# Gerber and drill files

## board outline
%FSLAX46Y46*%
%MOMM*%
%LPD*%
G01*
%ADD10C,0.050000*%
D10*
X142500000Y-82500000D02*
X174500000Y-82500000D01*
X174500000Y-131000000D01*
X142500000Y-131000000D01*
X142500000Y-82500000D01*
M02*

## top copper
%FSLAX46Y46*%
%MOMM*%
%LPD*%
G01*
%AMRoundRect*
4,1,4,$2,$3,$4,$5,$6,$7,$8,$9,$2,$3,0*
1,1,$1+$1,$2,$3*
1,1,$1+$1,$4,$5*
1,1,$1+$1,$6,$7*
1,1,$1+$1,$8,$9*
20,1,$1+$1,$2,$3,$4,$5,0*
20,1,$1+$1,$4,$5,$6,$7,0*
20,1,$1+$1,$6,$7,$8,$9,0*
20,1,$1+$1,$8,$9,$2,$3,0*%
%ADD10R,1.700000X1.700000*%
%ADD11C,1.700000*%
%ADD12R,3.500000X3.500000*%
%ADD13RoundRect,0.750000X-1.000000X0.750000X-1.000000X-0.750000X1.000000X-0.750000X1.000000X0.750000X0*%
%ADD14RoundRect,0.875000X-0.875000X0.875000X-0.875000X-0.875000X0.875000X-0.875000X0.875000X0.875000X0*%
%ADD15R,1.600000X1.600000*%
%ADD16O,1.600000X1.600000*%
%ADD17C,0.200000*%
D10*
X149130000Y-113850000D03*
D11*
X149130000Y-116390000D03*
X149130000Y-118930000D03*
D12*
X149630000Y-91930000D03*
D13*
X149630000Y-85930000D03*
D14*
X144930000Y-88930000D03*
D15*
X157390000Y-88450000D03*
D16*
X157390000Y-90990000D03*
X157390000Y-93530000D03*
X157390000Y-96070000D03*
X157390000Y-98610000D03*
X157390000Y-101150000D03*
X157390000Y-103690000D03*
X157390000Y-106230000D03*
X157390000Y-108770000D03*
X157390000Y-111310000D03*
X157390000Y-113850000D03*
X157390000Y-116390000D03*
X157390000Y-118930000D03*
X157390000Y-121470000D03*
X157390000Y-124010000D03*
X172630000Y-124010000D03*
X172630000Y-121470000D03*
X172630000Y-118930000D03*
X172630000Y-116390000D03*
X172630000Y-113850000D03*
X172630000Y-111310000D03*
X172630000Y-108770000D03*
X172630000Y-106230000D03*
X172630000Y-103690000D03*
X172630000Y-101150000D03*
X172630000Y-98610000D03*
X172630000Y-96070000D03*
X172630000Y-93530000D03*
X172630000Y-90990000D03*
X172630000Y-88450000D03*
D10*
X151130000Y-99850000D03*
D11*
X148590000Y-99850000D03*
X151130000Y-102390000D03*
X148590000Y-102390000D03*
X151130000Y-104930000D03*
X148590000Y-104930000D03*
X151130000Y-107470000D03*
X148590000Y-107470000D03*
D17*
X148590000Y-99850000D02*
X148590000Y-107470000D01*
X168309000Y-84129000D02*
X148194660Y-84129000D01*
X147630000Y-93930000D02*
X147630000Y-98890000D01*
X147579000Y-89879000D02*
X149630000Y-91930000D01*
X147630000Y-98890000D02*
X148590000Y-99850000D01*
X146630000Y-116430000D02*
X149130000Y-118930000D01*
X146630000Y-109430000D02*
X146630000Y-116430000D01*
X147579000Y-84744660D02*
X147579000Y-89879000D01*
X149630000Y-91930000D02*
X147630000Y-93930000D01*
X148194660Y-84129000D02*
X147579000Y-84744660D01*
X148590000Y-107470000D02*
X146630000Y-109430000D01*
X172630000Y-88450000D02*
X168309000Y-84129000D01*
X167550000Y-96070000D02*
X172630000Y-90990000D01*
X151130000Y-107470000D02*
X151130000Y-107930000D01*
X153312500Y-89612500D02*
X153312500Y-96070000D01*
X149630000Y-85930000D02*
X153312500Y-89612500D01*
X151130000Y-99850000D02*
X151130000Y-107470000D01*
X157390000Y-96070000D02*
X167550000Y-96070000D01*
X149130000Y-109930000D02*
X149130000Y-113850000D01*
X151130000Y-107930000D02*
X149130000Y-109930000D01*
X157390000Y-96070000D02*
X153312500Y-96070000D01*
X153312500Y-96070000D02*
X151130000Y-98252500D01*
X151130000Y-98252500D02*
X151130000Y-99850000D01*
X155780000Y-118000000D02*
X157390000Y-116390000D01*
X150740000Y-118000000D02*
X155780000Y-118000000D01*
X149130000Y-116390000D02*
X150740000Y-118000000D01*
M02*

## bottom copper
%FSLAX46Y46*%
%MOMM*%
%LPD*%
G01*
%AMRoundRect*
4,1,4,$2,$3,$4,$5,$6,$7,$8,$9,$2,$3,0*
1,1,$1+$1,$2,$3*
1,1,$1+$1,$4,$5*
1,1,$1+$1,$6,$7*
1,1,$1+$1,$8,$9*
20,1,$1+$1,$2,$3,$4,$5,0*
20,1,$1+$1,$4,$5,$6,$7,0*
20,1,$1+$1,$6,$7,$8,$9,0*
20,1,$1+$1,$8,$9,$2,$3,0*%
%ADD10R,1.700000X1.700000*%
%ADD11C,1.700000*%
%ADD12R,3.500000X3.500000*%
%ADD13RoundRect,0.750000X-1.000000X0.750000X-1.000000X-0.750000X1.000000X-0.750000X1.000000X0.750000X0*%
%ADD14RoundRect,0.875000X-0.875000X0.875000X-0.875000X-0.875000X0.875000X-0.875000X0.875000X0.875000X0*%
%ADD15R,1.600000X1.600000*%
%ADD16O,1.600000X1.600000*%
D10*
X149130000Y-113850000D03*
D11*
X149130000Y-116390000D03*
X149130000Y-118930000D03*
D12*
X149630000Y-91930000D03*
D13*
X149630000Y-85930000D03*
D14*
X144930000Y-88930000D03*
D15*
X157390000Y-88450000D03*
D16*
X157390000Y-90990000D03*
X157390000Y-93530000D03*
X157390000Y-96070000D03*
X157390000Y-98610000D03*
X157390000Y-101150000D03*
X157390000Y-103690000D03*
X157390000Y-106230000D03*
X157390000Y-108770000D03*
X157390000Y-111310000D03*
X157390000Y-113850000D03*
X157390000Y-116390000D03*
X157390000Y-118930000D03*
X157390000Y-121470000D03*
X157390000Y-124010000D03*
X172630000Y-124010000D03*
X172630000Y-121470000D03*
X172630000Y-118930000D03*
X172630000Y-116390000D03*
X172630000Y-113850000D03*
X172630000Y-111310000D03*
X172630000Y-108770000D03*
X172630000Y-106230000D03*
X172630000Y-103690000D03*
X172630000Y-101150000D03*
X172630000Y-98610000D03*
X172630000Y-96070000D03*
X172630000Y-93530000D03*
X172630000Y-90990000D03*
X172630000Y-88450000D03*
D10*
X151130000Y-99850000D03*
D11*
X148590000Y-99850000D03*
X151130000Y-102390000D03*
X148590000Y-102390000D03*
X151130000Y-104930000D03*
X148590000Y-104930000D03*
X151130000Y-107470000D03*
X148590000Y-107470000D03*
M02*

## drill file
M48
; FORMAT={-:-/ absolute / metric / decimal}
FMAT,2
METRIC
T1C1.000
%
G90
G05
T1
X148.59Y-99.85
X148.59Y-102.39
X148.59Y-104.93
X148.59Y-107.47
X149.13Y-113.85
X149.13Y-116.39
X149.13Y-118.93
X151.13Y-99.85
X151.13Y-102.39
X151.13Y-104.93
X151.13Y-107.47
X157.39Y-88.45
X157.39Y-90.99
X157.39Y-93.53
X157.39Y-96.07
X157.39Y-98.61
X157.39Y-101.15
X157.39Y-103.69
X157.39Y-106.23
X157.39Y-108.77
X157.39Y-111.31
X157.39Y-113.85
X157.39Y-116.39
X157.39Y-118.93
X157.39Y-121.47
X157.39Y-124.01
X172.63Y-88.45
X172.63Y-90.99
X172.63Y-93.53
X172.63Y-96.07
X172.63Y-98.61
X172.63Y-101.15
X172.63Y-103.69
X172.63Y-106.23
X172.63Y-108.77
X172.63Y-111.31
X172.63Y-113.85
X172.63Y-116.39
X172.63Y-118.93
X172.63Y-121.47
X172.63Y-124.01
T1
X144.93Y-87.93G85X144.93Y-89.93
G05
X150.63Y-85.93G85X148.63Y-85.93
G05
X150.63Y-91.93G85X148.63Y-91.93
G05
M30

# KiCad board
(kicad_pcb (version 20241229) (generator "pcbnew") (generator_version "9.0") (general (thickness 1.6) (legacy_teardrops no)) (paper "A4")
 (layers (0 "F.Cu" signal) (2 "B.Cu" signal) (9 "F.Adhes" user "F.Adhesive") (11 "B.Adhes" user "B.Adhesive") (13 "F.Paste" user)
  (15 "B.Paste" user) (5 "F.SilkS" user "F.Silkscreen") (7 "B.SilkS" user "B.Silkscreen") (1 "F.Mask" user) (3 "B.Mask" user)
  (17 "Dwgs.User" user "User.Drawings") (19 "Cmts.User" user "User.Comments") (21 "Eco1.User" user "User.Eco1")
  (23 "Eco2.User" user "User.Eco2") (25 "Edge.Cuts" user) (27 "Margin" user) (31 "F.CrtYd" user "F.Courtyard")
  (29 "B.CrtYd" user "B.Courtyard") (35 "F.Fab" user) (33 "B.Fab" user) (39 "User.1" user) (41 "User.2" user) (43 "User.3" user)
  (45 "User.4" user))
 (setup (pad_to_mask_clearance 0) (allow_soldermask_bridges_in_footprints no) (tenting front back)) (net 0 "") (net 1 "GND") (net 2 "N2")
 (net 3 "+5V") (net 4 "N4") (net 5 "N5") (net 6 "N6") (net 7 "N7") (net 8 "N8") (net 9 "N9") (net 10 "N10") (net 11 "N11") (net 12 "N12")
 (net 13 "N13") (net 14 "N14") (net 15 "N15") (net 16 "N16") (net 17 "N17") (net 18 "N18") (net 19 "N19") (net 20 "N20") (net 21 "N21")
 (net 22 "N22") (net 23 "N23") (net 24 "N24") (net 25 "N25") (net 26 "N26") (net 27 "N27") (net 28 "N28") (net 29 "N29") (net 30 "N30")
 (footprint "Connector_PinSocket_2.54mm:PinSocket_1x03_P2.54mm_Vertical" (layer "F.Cu") (at 149.13 113.85)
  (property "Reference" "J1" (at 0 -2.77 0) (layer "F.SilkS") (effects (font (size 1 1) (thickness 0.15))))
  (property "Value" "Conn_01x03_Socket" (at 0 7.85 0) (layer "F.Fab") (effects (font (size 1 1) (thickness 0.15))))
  (pad "1" thru_hole rect (at 0 0) (size 1.7 1.7) (drill 1) (layers "*.Cu" "*.Mask") (remove_unused_layers no) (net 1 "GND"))
  (pad "2" thru_hole circle (at 0 2.54) (size 1.7 1.7) (drill 1) (layers "*.Cu" "*.Mask") (remove_unused_layers no) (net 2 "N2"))
  (pad "3" thru_hole circle (at 0 5.08) (size 1.7 1.7) (drill 1) (layers "*.Cu" "*.Mask") (remove_unused_layers no) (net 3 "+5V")))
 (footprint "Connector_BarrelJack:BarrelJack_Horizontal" (layer "F.Cu") (at 149.63 91.93 -90)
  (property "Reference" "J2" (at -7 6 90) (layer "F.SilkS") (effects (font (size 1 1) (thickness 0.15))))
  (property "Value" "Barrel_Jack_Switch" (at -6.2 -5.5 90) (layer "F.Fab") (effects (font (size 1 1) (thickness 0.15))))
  (pad "1" thru_hole rect (at 0 0 270) (size 3.5 3.5) (drill oval 1 3) (layers "*.Cu" "*.Mask") (remove_unused_layers no) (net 3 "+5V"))
  (pad "2" thru_hole roundrect (at -6 0 270) (size 3 3.5) (drill oval 1 3) (layers "*.Cu" "*.Mask") (remove_unused_layers no)
   (roundrect_rratio 0.25) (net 1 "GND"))
  (pad "3" thru_hole roundrect (at -3 4.7 270) (size 3.5 3.5) (drill oval 3 1) (layers "*.Cu" "*.Mask") (remove_unused_layers no)
   (roundrect_rratio 0.25) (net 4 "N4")))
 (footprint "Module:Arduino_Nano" (layer "F.Cu") (at 157.39 88.45)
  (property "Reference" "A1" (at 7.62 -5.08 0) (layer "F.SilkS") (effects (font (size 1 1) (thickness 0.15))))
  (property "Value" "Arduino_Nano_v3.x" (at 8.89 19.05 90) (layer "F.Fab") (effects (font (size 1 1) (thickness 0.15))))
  (pad "1" thru_hole rect (at 0 0) (size 1.6 1.6) (drill 1) (layers "*.Cu" "*.Mask") (remove_unused_layers no) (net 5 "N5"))
  (pad "2" thru_hole oval (at 0 2.54) (size 1.6 1.6) (drill 1) (layers "*.Cu" "*.Mask") (remove_unused_layers no) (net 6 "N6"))
  (pad "3" thru_hole oval (at 0 5.08) (size 1.6 1.6) (drill 1) (layers "*.Cu" "*.Mask") (remove_unused_layers no) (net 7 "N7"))
  (pad "4" thru_hole oval (at 0 7.62) (size 1.6 1.6) (drill 1) (layers "*.Cu" "*.Mask") (remove_unused_layers no) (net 1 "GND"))
  (pad "5" thru_hole oval (at 0 10.16) (size 1.6 1.6) (drill 1) (layers "*.Cu" "*.Mask") (remove_unused_layers no) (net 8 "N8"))
  (pad "6" thru_hole oval (at 0 12.7) (size 1.6 1.6) (drill 1) (layers "*.Cu" "*.Mask") (remove_unused_layers no) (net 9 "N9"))
  (pad "7" thru_hole oval (at 0 15.24) (size 1.6 1.6) (drill 1) (layers "*.Cu" "*.Mask") (remove_unused_layers no) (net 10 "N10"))
  (pad "8" thru_hole oval (at 0 17.78) (size 1.6 1.6) (drill 1) (layers "*.Cu" "*.Mask") (remove_unused_layers no) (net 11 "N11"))
  (pad "9" thru_hole oval (at 0 20.32) (size 1.6 1.6) (drill 1) (layers "*.Cu" "*.Mask") (remove_unused_layers no) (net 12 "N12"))
  (pad "10" thru_hole oval (at 0 22.86) (size 1.6 1.6) (drill 1) (layers "*.Cu" "*.Mask") (remove_unused_layers no) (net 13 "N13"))
  (pad "11" thru_hole oval (at 0 25.4) (size 1.6 1.6) (drill 1) (layers "*.Cu" "*.Mask") (remove_unused_layers no) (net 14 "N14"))
  (pad "12" thru_hole oval (at 0 27.94) (size 1.6 1.6) (drill 1) (layers "*.Cu" "*.Mask") (remove_unused_layers no) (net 2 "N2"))
  (pad "13" thru_hole oval (at 0 30.48) (size 1.6 1.6) (drill 1) (layers "*.Cu" "*.Mask") (remove_unused_layers no) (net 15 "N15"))
  (pad "14" thru_hole oval (at 0 33.02) (size 1.6 1.6) (drill 1) (layers "*.Cu" "*.Mask") (remove_unused_layers no) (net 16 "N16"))
  (pad "15" thru_hole oval (at 0 35.56) (size 1.6 1.6) (drill 1) (layers "*.Cu" "*.Mask") (remove_unused_layers no) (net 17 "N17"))
  (pad "16" thru_hole oval (at 15.24 35.56) (size 1.6 1.6) (drill 1) (layers "*.Cu" "*.Mask") (remove_unused_layers no) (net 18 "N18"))
  (pad "17" thru_hole oval (at 15.24 33.02) (size 1.6 1.6) (drill 1) (layers "*.Cu" "*.Mask") (remove_unused_layers no) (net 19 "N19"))
  (pad "18" thru_hole oval (at 15.24 30.48) (size 1.6 1.6) (drill 1) (layers "*.Cu" "*.Mask") (remove_unused_layers no) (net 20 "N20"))
  (pad "19" thru_hole oval (at 15.24 27.94) (size 1.6 1.6) (drill 1) (layers "*.Cu" "*.Mask") (remove_unused_layers no) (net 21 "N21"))
  (pad "20" thru_hole oval (at 15.24 25.4) (size 1.6 1.6) (drill 1) (layers "*.Cu" "*.Mask") (remove_unused_layers no) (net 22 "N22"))
  (pad "21" thru_hole oval (at 15.24 22.86) (size 1.6 1.6) (drill 1) (layers "*.Cu" "*.Mask") (remove_unused_layers no) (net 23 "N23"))
  (pad "22" thru_hole oval (at 15.24 20.32) (size 1.6 1.6) (drill 1) (layers "*.Cu" "*.Mask") (remove_unused_layers no) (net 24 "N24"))
  (pad "23" thru_hole oval (at 15.24 17.78) (size 1.6 1.6) (drill 1) (layers "*.Cu" "*.Mask") (remove_unused_layers no) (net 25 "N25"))
  (pad "24" thru_hole oval (at 15.24 15.24) (size 1.6 1.6) (drill 1) (layers "*.Cu" "*.Mask") (remove_unused_layers no) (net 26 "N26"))
  (pad "25" thru_hole oval (at 15.24 12.7) (size 1.6 1.6) (drill 1) (layers "*.Cu" "*.Mask") (remove_unused_layers no) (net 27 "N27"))
  (pad "26" thru_hole oval (at 15.24 10.16) (size 1.6 1.6) (drill 1) (layers "*.Cu" "*.Mask") (remove_unused_layers no) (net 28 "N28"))
  (pad "27" thru_hole oval (at 15.24 7.62) (size 1.6 1.6) (drill 1) (layers "*.Cu" "*.Mask") (remove_unused_layers no) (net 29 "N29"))
  (pad "28" thru_hole oval (at 15.24 5.08) (size 1.6 1.6) (drill 1) (layers "*.Cu" "*.Mask") (remove_unused_layers no) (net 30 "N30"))
  (pad "29" thru_hole oval (at 15.24 2.54) (size 1.6 1.6) (drill 1) (layers "*.Cu" "*.Mask") (remove_unused_layers no) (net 1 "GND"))
  (pad "30" thru_hole oval (at 15.24 0) (size 1.6 1.6) (drill 1) (layers "*.Cu" "*.Mask") (remove_unused_layers no) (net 3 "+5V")))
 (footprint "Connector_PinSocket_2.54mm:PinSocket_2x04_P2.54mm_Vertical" (layer "F.Cu") (at 151.13 99.85)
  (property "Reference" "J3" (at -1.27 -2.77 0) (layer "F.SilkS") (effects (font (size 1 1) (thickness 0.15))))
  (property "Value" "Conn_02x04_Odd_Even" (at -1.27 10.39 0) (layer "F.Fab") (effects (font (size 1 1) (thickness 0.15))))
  (pad "1" thru_hole rect (at 0 0) (size 1.7 1.7) (drill 1) (layers "*.Cu" "*.Mask") (remove_unused_layers no) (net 1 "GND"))
  (pad "2" thru_hole circle (at -2.54 0) (size 1.7 1.7) (drill 1) (layers "*.Cu" "*.Mask") (remove_unused_layers no) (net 3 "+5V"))
  (pad "3" thru_hole circle (at 0 2.54) (size 1.7 1.7) (drill 1) (layers "*.Cu" "*.Mask") (remove_unused_layers no) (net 1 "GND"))
  (pad "4" thru_hole circle (at -2.54 2.54) (size 1.7 1.7) (drill 1) (layers "*.Cu" "*.Mask") (remove_unused_layers no) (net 3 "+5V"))
  (pad "5" thru_hole circle (at 0 5.08) (size 1.7 1.7) (drill 1) (layers "*.Cu" "*.Mask") (remove_unused_layers no) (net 1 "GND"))
  (pad "6" thru_hole circle (at -2.54 5.08) (size 1.7 1.7) (drill 1) (layers "*.Cu" "*.Mask") (remove_unused_layers no) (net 3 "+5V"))
  (pad "7" thru_hole circle (at 0 7.62) (size 1.7 1.7) (drill 1) (layers "*.Cu" "*.Mask") (remove_unused_layers no) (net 1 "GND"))
  (pad "8" thru_hole circle (at -2.54 7.62) (size 1.7 1.7) (drill 1) (layers "*.Cu" "*.Mask") (remove_unused_layers no) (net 3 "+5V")))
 (gr_rect (start 142.5 82.5) (end 174.5 131) (stroke (width 0.05) (type default)) (fill no) (layer "Edge.Cuts"))
 (segment (start 148.59 99.85) (end 148.59 107.47) (width 0.2) (layer "F.Cu") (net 3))
 (segment (start 168.309 84.129) (end 148.19466 84.129) (width 0.2) (layer "F.Cu") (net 3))
 (segment (start 147.63 93.93) (end 147.63 98.89) (width 0.2) (layer "F.Cu") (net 3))
 (segment (start 147.579 89.879) (end 149.63 91.93) (width 0.2) (layer "F.Cu") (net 3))
 (segment (start 147.63 98.89) (end 148.59 99.85) (width 0.2) (layer "F.Cu") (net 3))
 (segment (start 146.63 116.43) (end 149.13 118.93) (width 0.2) (layer "F.Cu") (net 3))
 (segment (start 146.63 109.43) (end 146.63 116.43) (width 0.2) (layer "F.Cu") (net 3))
 (segment (start 147.579 84.74466) (end 147.579 89.879) (width 0.2) (layer "F.Cu") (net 3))
 (segment (start 149.63 91.93) (end 147.63 93.93) (width 0.2) (layer "F.Cu") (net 3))
 (segment (start 148.19466 84.129) (end 147.579 84.74466) (width 0.2) (layer "F.Cu") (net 3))
 (segment (start 148.59 107.47) (end 146.63 109.43) (width 0.2) (layer "F.Cu") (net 3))
 (segment (start 172.63 88.45) (end 168.309 84.129) (width 0.2) (layer "F.Cu") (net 3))
 (segment (start 167.55 96.07) (end 172.63 90.99) (width 0.2) (layer "F.Cu") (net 1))
 (segment (start 151.13 107.47) (end 151.13 107.93) (width 0.2) (layer "F.Cu") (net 1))
 (segment (start 153.3125 89.6125) (end 153.3125 96.07) (width 0.2) (layer "F.Cu") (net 1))
 (segment (start 149.63 85.93) (end 153.3125 89.6125) (width 0.2) (layer "F.Cu") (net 1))
 (segment (start 151.13 99.85) (end 151.13 107.47) (width 0.2) (layer "F.Cu") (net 1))
 (segment (start 157.39 96.07) (end 167.55 96.07) (width 0.2) (layer "F.Cu") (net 1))
 (segment (start 149.13 109.93) (end 149.13 113.85) (width 0.2) (layer "F.Cu") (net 1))
 (segment (start 151.13 107.93) (end 149.13 109.93) (width 0.2) (layer "F.Cu") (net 1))
 (segment (start 157.39 96.07) (end 153.3125 96.07) (width 0.2) (layer "F.Cu") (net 1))
 (segment (start 153.3125 96.07) (end 151.13 98.2525) (width 0.2) (layer "F.Cu") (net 1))
 (segment (start 151.13 98.2525) (end 151.13 99.85) (width 0.2) (layer "F.Cu") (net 1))
 (segment (start 155.78 118) (end 157.39 116.39) (width 0.2) (layer "F.Cu") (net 2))
 (segment (start 150.74 118) (end 155.78 118) (width 0.2) (layer "F.Cu") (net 2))
 (segment (start 149.13 116.39) (end 150.74 118) (width 0.2) (layer "F.Cu") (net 2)))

